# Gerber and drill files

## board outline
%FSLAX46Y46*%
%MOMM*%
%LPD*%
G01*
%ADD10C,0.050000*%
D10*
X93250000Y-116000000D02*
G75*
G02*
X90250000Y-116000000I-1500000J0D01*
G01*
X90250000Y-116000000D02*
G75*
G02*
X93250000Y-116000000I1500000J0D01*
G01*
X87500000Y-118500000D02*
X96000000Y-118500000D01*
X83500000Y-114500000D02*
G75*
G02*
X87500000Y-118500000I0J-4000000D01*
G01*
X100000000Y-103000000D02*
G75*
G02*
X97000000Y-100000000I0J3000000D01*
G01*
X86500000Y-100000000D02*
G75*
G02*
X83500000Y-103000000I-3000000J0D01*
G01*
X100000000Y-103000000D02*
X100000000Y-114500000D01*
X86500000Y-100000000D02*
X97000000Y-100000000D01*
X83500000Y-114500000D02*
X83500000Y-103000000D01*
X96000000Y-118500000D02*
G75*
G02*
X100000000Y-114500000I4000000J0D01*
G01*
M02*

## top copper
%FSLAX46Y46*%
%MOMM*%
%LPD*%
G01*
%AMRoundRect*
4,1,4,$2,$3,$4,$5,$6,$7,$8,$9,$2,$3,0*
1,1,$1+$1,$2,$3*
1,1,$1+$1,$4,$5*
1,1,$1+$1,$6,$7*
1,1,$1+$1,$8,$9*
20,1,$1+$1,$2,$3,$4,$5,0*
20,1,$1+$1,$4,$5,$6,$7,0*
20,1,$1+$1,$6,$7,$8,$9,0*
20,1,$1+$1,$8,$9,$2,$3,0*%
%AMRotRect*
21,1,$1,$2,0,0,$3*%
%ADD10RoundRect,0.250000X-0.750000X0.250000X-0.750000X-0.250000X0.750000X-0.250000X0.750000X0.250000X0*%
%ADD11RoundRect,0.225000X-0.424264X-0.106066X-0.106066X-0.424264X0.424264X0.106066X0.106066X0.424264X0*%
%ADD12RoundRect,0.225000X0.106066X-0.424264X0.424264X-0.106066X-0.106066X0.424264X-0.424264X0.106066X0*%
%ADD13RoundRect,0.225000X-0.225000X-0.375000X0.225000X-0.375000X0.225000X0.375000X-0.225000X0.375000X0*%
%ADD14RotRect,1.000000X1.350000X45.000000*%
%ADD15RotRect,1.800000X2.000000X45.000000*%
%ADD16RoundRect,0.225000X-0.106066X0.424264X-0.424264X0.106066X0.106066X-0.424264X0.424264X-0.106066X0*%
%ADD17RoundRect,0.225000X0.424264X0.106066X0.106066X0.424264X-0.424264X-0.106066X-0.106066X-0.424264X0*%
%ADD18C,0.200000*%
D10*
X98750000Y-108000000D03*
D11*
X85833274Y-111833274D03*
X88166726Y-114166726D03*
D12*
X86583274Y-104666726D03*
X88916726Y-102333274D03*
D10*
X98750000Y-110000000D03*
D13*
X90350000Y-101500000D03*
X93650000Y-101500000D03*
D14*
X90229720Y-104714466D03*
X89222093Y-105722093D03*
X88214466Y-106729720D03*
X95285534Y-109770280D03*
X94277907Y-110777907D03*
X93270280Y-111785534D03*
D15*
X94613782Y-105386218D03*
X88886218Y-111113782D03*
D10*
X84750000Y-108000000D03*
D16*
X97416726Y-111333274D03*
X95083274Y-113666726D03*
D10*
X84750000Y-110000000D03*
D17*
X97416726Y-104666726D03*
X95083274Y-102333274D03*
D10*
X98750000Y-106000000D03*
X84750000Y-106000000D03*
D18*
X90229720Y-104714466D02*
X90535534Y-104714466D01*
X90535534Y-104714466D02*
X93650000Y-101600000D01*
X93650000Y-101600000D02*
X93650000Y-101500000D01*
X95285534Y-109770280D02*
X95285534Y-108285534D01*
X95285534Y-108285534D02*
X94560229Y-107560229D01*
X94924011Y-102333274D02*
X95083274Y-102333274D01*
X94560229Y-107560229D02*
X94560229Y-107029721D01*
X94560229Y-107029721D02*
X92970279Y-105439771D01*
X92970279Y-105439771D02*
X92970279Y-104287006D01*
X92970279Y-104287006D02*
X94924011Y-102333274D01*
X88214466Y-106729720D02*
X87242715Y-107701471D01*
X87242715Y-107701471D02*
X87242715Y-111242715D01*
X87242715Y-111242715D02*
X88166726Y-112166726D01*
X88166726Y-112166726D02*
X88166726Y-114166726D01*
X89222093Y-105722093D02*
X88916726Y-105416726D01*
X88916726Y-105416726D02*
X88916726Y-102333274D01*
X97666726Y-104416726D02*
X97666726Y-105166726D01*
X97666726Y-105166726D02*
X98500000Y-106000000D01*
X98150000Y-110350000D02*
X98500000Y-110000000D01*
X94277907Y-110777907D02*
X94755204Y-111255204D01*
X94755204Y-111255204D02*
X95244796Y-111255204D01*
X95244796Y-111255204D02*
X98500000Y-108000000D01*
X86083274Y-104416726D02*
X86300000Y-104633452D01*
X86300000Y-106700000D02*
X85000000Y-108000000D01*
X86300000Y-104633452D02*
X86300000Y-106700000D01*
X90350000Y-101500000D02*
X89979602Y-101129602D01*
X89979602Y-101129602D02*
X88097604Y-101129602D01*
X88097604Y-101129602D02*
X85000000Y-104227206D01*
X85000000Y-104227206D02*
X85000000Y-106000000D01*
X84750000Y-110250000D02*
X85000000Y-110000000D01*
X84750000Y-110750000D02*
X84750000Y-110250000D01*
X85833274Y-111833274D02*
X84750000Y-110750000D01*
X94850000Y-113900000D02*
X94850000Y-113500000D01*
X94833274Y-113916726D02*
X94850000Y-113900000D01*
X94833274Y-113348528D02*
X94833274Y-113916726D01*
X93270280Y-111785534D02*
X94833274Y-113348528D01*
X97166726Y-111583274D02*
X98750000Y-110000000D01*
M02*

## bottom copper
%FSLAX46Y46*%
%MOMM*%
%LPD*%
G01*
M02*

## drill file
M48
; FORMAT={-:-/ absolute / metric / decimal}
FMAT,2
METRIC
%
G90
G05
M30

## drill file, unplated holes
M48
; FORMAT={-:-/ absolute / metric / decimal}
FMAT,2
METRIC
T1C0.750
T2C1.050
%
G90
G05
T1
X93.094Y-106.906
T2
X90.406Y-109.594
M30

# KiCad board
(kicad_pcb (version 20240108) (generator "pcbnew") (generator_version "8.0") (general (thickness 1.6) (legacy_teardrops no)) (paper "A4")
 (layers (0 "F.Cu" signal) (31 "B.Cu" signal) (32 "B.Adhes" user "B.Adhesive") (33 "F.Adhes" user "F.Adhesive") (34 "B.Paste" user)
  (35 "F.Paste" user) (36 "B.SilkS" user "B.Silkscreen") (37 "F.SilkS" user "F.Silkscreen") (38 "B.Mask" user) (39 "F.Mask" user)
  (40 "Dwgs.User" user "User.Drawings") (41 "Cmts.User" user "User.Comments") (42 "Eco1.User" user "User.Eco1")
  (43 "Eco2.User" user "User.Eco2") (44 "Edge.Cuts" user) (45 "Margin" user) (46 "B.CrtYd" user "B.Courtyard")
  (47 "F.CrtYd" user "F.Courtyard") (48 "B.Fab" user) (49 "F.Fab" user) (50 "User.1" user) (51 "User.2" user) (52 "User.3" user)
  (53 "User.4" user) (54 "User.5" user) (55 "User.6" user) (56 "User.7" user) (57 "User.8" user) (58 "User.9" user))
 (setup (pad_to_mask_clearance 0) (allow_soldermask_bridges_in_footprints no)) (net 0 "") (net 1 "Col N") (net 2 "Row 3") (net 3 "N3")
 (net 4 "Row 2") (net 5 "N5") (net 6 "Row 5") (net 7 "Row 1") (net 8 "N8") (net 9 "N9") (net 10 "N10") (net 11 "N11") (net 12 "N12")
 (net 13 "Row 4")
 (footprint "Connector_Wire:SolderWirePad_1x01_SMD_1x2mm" (layer "F.Cu") (at 98.75 108 -90)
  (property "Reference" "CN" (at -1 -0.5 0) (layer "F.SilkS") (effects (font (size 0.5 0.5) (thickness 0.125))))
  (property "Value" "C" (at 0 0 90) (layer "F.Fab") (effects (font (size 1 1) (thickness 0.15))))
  (pad "1" smd roundrect (at 0 0 270) (size 1 2) (layers "F.Cu" "F.Paste" "F.Mask") (roundrect_rratio 0.25) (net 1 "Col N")))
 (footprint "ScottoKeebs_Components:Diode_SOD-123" (layer "F.Cu") (at 87 113 -45)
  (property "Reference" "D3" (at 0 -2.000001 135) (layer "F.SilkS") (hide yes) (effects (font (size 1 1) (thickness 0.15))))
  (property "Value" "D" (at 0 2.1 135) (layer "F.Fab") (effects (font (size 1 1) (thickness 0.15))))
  (pad "1" smd roundrect (at -1.65 0 315) (size 0.9 1.2) (layers "F.Cu" "F.Paste" "F.Mask") (roundrect_rratio 0.25) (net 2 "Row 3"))
  (pad "2" smd roundrect (at 1.65 0 315) (size 0.9 1.2) (layers "F.Cu" "F.Paste" "F.Mask") (roundrect_rratio 0.25) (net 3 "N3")))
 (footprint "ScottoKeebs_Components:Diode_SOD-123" (layer "F.Cu") (at 87.75 103.5 45)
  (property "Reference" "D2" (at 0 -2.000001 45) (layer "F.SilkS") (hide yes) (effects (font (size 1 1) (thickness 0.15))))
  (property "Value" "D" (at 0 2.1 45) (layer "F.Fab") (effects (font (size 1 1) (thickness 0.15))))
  (pad "1" smd roundrect (at -1.65 0 45) (size 0.9 1.2) (layers "F.Cu" "F.Paste" "F.Mask") (roundrect_rratio 0.25) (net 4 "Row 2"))
  (pad "2" smd roundrect (at 1.65 0 45) (size 0.9 1.2) (layers "F.Cu" "F.Paste" "F.Mask") (roundrect_rratio 0.25) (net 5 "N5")))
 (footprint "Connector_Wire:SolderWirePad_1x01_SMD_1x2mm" (layer "F.Cu") (at 98.75 110 -90)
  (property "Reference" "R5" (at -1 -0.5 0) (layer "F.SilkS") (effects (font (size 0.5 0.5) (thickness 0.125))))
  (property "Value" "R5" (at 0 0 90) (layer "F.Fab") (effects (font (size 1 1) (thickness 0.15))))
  (pad "1" smd roundrect (at 0 0 270) (size 1 2) (layers "F.Cu" "F.Paste" "F.Mask") (roundrect_rratio 0.25) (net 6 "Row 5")))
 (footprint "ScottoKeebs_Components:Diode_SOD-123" (layer "F.Cu") (at 92 101.5)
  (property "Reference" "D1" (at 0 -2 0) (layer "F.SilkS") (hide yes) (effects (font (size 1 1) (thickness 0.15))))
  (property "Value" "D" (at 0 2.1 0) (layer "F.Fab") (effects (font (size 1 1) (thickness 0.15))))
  (pad "1" smd roundrect (at -1.65 0) (size 0.9 1.2) (layers "F.Cu" "F.Paste" "F.Mask") (roundrect_rratio 0.25) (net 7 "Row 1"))
  (pad "2" smd roundrect (at 1.65 0) (size 0.9 1.2) (layers "F.Cu" "F.Paste" "F.Mask") (roundrect_rratio 0.25) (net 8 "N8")))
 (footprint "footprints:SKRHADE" (layer "F.Cu") (at 91.75 108.25 -45)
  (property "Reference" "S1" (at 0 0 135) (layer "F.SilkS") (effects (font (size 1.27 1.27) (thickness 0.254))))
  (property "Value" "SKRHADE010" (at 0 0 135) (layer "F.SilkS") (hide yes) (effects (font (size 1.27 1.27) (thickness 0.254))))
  (pad "" np_thru_hole circle (at 0 -1.9 315) (size 0.75 0.75) (drill 0.75) (layers "*.Cu" "*.Mask"))
  (pad "" np_thru_hole circle (at 0 1.9 315) (size 1.05 1.05) (drill 1.05) (layers "*.Cu" "*.Mask"))
  (pad "1" smd rect (at -3.575 -1.425 45) (size 1 1.35) (layers "F.Cu" "F.Paste" "F.Mask") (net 8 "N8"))
  (pad "2" smd rect (at -3.575 0 45) (size 1 1.35) (layers "F.Cu" "F.Paste" "F.Mask") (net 5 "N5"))
  (pad "3" smd rect (at -3.575 1.425 45) (size 1 1.35) (layers "F.Cu" "F.Paste" "F.Mask") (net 3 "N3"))
  (pad "4" smd rect (at 3.575 -1.425 45) (size 1 1.35) (layers "F.Cu" "F.Paste" "F.Mask") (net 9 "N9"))
  (pad "5" smd rect (at 3.575 0 45) (size 1 1.35) (layers "F.Cu" "F.Paste" "F.Mask") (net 1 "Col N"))
  (pad "6" smd rect (at 3.575 1.425 45) (size 1 1.35) (layers "F.Cu" "F.Paste" "F.Mask") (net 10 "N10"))
  (pad "MP1" smd rect (at 0 -4.049999 45) (size 1.8 2) (layers "F.Cu" "F.Paste" "F.Mask") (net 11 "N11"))
  (pad "MP2" smd rect (at 0 4.049999 45) (size 1.8 2) (layers "F.Cu" "F.Paste" "F.Mask") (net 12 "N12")))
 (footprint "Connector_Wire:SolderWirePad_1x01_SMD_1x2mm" (layer "F.Cu") (at 84.75 108 -90)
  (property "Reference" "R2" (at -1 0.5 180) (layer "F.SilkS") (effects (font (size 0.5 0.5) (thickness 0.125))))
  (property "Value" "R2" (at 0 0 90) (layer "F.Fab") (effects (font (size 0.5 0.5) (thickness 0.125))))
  (pad "1" smd roundrect (at 0 0 270) (size 1 2) (layers "F.Cu" "F.Paste" "F.Mask") (roundrect_rratio 0.25) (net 4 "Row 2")))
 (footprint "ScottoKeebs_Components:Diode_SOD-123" (layer "F.Cu") (at 96.25 112.5 -135)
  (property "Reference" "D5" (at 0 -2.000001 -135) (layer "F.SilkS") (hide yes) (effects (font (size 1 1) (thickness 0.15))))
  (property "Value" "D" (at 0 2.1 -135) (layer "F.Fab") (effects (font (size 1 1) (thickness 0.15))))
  (pad "1" smd roundrect (at -1.65 0 225) (size 0.9 1.2) (layers "F.Cu" "F.Paste" "F.Mask") (roundrect_rratio 0.25) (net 6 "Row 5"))
  (pad "2" smd roundrect (at 1.65 0 225) (size 0.9 1.2) (layers "F.Cu" "F.Paste" "F.Mask") (roundrect_rratio 0.25) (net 10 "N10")))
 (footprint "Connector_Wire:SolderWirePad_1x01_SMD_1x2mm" (layer "F.Cu") (at 84.75 110 -90)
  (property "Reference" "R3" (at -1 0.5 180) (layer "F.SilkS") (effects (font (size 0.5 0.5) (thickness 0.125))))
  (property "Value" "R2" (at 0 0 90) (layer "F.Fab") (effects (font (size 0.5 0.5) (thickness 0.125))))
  (pad "1" smd roundrect (at 0 0 270) (size 1 2) (layers "F.Cu" "F.Paste" "F.Mask") (roundrect_rratio 0.25) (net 2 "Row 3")))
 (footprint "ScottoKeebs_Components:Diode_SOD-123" (layer "F.Cu") (at 96.25 103.5 135)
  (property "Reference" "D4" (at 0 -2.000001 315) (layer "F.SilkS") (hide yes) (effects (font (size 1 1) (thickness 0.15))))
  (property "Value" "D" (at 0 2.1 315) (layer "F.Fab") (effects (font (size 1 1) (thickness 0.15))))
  (pad "1" smd roundrect (at -1.65 0 135) (size 0.9 1.2) (layers "F.Cu" "F.Paste" "F.Mask") (roundrect_rratio 0.25) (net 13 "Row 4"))
  (pad "2" smd roundrect (at 1.65 0 135) (size 0.9 1.2) (layers "F.Cu" "F.Paste" "F.Mask") (roundrect_rratio 0.25) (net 9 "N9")))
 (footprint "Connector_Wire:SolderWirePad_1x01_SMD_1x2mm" (layer "F.Cu") (at 98.75 106 -90)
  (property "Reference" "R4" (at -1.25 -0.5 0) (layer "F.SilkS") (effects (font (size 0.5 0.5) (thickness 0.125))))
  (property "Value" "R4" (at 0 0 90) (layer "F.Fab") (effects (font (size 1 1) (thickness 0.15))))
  (pad "1" smd roundrect (at 0 0 270) (size 1 2) (layers "F.Cu" "F.Paste" "F.Mask") (roundrect_rratio 0.25) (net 13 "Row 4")))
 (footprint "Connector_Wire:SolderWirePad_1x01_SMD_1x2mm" (layer "F.Cu") (at 84.75 106 -90)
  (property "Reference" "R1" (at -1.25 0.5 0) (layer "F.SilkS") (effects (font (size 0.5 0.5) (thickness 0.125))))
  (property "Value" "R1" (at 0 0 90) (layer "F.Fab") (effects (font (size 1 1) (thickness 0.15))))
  (pad "1" smd roundrect (at 0 0 270) (size 1 2) (layers "F.Cu" "F.Paste" "F.Mask") (roundrect_rratio 0.25) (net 7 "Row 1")))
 (gr_arc (start 83.5 114.5) (mid 86.328427 115.671573) (end 87.5 118.5) (stroke (width 0.05) (type default)) (layer "Edge.Cuts"))
 (gr_arc (start 100 103) (mid 97.87868 102.12132) (end 97 100) (stroke (width 0.05) (type default)) (layer "Edge.Cuts"))
 (gr_arc (start 86.5 100) (mid 85.62132 102.12132) (end 83.5 103) (stroke (width 0.05) (type default)) (layer "Edge.Cuts"))
 (gr_line (start 100 103) (end 100 114.5) (stroke (width 0.05) (type default)) (layer "Edge.Cuts"))
 (gr_line (start 86.5 100) (end 97 100) (stroke (width 0.05) (type default)) (layer "Edge.Cuts"))
 (gr_line (start 83.5 114.5) (end 83.5 103) (stroke (width 0.05) (type default)) (layer "Edge.Cuts"))
 (gr_circle (center 91.75 116) (end 93.25 116) (stroke (width 0.05) (type default)) (fill none) (layer "Edge.Cuts"))
 (gr_arc (start 96 118.5) (mid 97.171573 115.671573) (end 100 114.5) (stroke (width 0.05) (type default)) (layer "Edge.Cuts"))
 (gr_line (start 87.5 118.5) (end 96 118.5) (stroke (width 0.05) (type default)) (layer "Edge.Cuts"))
 (segment (start 90.35 101.5) (end 89.979602 101.129602) (width 0.2) (layer "F.Cu") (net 7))
 (segment (start 89.979602 101.129602) (end 88.097604 101.129602) (width 0.2) (layer "F.Cu") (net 7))
 (segment (start 85 104.227206) (end 85 106) (width 0.2) (layer "F.Cu") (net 7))
 (segment (start 88.097604 101.129602) (end 85 104.227206) (width 0.2) (layer "F.Cu") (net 7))
 (segment (start 93.65 101.6) (end 93.65 101.5) (width 0.2) (layer "F.Cu") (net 8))
 (segment (start 90.22972 104.714466) (end 90.535534 104.714466) (width 0.2) (layer "F.Cu") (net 8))
 (segment (start 90.535534 104.714466) (end 93.65 101.6) (width 0.2) (layer "F.Cu") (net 8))
 (segment (start 88.916726 105.416726) (end 88.916726 102.333274) (width 0.2) (layer "F.Cu") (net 5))
 (segment (start 89.222093 105.722093) (end 88.916726 105.416726) (width 0.2) (layer "F.Cu") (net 5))
 (segment (start 86.3 104.633452) (end 86.3 106.7) (width 0.2) (layer "F.Cu") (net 4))
 (segment (start 86.083274 104.416726) (end 86.3 104.633452) (width 0.2) (layer "F.Cu") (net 4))
 (segment (start 86.3 106.7) (end 85 108) (width 0.2) (layer "F.Cu") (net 4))
 (segment (start 88.214466 106.72972) (end 87.242715 107.701471) (width 0.2) (layer "F.Cu") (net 3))
 (segment (start 87.242715 111.242715) (end 88.166726 112.166726) (width 0.2) (layer "F.Cu") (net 3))
 (segment (start 88.166726 112.166726) (end 88.166726 114.166726) (width 0.2) (layer "F.Cu") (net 3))
 (segment (start 87.242715 107.701471) (end 87.242715 111.242715) (width 0.2) (layer "F.Cu") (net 3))
 (segment (start 85.833274 111.833274) (end 84.75 110.75) (width 0.2) (layer "F.Cu") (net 2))
 (segment (start 84.75 110.25) (end 85 110) (width 0.2) (layer "F.Cu") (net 2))
 (segment (start 84.75 110.75) (end 84.75 110.25) (width 0.2) (layer "F.Cu") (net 2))
 (segment (start 94.560229 107.560229) (end 94.560229 107.029721) (width 0.2) (layer "F.Cu") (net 9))
 (segment (start 92.970279 105.439771) (end 92.970279 104.287006) (width 0.2) (layer "F.Cu") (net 9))
 (segment (start 94.560229 107.029721) (end 92.970279 105.439771) (width 0.2) (layer "F.Cu") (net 9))
 (segment (start 95.285534 108.285534) (end 94.560229 107.560229) (width 0.2) (layer "F.Cu") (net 9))
 (segment (start 92.970279 104.287006) (end 94.924011 102.333274) (width 0.2) (layer "F.Cu") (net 9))
 (segment (start 94.924011 102.333274) (end 95.083274 102.333274) (width 0.2) (layer "F.Cu") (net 9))
 (segment (start 95.285534 109.77028) (end 95.285534 108.285534) (width 0.2) (layer "F.Cu") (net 9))
 (segment (start 97.666726 105.166726) (end 98.5 106) (width 0.2) (layer "F.Cu") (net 13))
 (segment (start 97.666726 104.416726) (end 97.666726 105.166726) (width 0.2) (layer "F.Cu") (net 13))
 (segment (start 94.85 113.9) (end 94.85 113.5) (width 0.2) (layer "F.Cu") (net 10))
 (segment (start 94.833274 113.916726) (end 94.85 113.9) (width 0.2) (layer "F.Cu") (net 10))
 (segment (start 94.833274 113.348528) (end 94.833274 113.916726) (width 0.2) (layer "F.Cu") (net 10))
 (segment (start 93.27028 111.785534) (end 94.833274 113.348528) (width 0.2) (layer "F.Cu") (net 10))
 (segment (start 98.15 110.35) (end 98.5 110) (width 0.2) (layer "F.Cu") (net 6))
 (segment (start 97.166726 111.583274) (end 98.75 110) (width 0.2) (layer "F.Cu") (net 6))
 (segment (start 94.277907 110.777907) (end 94.755204 111.255204) (width 0.2) (layer "F.Cu") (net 1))
 (segment (start 94.755204 111.255204) (end 95.244796 111.255204) (width 0.2) (layer "F.Cu") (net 1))
 (segment (start 95.244796 111.255204) (end 98.5 108) (width 0.2) (layer "F.Cu") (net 1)))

